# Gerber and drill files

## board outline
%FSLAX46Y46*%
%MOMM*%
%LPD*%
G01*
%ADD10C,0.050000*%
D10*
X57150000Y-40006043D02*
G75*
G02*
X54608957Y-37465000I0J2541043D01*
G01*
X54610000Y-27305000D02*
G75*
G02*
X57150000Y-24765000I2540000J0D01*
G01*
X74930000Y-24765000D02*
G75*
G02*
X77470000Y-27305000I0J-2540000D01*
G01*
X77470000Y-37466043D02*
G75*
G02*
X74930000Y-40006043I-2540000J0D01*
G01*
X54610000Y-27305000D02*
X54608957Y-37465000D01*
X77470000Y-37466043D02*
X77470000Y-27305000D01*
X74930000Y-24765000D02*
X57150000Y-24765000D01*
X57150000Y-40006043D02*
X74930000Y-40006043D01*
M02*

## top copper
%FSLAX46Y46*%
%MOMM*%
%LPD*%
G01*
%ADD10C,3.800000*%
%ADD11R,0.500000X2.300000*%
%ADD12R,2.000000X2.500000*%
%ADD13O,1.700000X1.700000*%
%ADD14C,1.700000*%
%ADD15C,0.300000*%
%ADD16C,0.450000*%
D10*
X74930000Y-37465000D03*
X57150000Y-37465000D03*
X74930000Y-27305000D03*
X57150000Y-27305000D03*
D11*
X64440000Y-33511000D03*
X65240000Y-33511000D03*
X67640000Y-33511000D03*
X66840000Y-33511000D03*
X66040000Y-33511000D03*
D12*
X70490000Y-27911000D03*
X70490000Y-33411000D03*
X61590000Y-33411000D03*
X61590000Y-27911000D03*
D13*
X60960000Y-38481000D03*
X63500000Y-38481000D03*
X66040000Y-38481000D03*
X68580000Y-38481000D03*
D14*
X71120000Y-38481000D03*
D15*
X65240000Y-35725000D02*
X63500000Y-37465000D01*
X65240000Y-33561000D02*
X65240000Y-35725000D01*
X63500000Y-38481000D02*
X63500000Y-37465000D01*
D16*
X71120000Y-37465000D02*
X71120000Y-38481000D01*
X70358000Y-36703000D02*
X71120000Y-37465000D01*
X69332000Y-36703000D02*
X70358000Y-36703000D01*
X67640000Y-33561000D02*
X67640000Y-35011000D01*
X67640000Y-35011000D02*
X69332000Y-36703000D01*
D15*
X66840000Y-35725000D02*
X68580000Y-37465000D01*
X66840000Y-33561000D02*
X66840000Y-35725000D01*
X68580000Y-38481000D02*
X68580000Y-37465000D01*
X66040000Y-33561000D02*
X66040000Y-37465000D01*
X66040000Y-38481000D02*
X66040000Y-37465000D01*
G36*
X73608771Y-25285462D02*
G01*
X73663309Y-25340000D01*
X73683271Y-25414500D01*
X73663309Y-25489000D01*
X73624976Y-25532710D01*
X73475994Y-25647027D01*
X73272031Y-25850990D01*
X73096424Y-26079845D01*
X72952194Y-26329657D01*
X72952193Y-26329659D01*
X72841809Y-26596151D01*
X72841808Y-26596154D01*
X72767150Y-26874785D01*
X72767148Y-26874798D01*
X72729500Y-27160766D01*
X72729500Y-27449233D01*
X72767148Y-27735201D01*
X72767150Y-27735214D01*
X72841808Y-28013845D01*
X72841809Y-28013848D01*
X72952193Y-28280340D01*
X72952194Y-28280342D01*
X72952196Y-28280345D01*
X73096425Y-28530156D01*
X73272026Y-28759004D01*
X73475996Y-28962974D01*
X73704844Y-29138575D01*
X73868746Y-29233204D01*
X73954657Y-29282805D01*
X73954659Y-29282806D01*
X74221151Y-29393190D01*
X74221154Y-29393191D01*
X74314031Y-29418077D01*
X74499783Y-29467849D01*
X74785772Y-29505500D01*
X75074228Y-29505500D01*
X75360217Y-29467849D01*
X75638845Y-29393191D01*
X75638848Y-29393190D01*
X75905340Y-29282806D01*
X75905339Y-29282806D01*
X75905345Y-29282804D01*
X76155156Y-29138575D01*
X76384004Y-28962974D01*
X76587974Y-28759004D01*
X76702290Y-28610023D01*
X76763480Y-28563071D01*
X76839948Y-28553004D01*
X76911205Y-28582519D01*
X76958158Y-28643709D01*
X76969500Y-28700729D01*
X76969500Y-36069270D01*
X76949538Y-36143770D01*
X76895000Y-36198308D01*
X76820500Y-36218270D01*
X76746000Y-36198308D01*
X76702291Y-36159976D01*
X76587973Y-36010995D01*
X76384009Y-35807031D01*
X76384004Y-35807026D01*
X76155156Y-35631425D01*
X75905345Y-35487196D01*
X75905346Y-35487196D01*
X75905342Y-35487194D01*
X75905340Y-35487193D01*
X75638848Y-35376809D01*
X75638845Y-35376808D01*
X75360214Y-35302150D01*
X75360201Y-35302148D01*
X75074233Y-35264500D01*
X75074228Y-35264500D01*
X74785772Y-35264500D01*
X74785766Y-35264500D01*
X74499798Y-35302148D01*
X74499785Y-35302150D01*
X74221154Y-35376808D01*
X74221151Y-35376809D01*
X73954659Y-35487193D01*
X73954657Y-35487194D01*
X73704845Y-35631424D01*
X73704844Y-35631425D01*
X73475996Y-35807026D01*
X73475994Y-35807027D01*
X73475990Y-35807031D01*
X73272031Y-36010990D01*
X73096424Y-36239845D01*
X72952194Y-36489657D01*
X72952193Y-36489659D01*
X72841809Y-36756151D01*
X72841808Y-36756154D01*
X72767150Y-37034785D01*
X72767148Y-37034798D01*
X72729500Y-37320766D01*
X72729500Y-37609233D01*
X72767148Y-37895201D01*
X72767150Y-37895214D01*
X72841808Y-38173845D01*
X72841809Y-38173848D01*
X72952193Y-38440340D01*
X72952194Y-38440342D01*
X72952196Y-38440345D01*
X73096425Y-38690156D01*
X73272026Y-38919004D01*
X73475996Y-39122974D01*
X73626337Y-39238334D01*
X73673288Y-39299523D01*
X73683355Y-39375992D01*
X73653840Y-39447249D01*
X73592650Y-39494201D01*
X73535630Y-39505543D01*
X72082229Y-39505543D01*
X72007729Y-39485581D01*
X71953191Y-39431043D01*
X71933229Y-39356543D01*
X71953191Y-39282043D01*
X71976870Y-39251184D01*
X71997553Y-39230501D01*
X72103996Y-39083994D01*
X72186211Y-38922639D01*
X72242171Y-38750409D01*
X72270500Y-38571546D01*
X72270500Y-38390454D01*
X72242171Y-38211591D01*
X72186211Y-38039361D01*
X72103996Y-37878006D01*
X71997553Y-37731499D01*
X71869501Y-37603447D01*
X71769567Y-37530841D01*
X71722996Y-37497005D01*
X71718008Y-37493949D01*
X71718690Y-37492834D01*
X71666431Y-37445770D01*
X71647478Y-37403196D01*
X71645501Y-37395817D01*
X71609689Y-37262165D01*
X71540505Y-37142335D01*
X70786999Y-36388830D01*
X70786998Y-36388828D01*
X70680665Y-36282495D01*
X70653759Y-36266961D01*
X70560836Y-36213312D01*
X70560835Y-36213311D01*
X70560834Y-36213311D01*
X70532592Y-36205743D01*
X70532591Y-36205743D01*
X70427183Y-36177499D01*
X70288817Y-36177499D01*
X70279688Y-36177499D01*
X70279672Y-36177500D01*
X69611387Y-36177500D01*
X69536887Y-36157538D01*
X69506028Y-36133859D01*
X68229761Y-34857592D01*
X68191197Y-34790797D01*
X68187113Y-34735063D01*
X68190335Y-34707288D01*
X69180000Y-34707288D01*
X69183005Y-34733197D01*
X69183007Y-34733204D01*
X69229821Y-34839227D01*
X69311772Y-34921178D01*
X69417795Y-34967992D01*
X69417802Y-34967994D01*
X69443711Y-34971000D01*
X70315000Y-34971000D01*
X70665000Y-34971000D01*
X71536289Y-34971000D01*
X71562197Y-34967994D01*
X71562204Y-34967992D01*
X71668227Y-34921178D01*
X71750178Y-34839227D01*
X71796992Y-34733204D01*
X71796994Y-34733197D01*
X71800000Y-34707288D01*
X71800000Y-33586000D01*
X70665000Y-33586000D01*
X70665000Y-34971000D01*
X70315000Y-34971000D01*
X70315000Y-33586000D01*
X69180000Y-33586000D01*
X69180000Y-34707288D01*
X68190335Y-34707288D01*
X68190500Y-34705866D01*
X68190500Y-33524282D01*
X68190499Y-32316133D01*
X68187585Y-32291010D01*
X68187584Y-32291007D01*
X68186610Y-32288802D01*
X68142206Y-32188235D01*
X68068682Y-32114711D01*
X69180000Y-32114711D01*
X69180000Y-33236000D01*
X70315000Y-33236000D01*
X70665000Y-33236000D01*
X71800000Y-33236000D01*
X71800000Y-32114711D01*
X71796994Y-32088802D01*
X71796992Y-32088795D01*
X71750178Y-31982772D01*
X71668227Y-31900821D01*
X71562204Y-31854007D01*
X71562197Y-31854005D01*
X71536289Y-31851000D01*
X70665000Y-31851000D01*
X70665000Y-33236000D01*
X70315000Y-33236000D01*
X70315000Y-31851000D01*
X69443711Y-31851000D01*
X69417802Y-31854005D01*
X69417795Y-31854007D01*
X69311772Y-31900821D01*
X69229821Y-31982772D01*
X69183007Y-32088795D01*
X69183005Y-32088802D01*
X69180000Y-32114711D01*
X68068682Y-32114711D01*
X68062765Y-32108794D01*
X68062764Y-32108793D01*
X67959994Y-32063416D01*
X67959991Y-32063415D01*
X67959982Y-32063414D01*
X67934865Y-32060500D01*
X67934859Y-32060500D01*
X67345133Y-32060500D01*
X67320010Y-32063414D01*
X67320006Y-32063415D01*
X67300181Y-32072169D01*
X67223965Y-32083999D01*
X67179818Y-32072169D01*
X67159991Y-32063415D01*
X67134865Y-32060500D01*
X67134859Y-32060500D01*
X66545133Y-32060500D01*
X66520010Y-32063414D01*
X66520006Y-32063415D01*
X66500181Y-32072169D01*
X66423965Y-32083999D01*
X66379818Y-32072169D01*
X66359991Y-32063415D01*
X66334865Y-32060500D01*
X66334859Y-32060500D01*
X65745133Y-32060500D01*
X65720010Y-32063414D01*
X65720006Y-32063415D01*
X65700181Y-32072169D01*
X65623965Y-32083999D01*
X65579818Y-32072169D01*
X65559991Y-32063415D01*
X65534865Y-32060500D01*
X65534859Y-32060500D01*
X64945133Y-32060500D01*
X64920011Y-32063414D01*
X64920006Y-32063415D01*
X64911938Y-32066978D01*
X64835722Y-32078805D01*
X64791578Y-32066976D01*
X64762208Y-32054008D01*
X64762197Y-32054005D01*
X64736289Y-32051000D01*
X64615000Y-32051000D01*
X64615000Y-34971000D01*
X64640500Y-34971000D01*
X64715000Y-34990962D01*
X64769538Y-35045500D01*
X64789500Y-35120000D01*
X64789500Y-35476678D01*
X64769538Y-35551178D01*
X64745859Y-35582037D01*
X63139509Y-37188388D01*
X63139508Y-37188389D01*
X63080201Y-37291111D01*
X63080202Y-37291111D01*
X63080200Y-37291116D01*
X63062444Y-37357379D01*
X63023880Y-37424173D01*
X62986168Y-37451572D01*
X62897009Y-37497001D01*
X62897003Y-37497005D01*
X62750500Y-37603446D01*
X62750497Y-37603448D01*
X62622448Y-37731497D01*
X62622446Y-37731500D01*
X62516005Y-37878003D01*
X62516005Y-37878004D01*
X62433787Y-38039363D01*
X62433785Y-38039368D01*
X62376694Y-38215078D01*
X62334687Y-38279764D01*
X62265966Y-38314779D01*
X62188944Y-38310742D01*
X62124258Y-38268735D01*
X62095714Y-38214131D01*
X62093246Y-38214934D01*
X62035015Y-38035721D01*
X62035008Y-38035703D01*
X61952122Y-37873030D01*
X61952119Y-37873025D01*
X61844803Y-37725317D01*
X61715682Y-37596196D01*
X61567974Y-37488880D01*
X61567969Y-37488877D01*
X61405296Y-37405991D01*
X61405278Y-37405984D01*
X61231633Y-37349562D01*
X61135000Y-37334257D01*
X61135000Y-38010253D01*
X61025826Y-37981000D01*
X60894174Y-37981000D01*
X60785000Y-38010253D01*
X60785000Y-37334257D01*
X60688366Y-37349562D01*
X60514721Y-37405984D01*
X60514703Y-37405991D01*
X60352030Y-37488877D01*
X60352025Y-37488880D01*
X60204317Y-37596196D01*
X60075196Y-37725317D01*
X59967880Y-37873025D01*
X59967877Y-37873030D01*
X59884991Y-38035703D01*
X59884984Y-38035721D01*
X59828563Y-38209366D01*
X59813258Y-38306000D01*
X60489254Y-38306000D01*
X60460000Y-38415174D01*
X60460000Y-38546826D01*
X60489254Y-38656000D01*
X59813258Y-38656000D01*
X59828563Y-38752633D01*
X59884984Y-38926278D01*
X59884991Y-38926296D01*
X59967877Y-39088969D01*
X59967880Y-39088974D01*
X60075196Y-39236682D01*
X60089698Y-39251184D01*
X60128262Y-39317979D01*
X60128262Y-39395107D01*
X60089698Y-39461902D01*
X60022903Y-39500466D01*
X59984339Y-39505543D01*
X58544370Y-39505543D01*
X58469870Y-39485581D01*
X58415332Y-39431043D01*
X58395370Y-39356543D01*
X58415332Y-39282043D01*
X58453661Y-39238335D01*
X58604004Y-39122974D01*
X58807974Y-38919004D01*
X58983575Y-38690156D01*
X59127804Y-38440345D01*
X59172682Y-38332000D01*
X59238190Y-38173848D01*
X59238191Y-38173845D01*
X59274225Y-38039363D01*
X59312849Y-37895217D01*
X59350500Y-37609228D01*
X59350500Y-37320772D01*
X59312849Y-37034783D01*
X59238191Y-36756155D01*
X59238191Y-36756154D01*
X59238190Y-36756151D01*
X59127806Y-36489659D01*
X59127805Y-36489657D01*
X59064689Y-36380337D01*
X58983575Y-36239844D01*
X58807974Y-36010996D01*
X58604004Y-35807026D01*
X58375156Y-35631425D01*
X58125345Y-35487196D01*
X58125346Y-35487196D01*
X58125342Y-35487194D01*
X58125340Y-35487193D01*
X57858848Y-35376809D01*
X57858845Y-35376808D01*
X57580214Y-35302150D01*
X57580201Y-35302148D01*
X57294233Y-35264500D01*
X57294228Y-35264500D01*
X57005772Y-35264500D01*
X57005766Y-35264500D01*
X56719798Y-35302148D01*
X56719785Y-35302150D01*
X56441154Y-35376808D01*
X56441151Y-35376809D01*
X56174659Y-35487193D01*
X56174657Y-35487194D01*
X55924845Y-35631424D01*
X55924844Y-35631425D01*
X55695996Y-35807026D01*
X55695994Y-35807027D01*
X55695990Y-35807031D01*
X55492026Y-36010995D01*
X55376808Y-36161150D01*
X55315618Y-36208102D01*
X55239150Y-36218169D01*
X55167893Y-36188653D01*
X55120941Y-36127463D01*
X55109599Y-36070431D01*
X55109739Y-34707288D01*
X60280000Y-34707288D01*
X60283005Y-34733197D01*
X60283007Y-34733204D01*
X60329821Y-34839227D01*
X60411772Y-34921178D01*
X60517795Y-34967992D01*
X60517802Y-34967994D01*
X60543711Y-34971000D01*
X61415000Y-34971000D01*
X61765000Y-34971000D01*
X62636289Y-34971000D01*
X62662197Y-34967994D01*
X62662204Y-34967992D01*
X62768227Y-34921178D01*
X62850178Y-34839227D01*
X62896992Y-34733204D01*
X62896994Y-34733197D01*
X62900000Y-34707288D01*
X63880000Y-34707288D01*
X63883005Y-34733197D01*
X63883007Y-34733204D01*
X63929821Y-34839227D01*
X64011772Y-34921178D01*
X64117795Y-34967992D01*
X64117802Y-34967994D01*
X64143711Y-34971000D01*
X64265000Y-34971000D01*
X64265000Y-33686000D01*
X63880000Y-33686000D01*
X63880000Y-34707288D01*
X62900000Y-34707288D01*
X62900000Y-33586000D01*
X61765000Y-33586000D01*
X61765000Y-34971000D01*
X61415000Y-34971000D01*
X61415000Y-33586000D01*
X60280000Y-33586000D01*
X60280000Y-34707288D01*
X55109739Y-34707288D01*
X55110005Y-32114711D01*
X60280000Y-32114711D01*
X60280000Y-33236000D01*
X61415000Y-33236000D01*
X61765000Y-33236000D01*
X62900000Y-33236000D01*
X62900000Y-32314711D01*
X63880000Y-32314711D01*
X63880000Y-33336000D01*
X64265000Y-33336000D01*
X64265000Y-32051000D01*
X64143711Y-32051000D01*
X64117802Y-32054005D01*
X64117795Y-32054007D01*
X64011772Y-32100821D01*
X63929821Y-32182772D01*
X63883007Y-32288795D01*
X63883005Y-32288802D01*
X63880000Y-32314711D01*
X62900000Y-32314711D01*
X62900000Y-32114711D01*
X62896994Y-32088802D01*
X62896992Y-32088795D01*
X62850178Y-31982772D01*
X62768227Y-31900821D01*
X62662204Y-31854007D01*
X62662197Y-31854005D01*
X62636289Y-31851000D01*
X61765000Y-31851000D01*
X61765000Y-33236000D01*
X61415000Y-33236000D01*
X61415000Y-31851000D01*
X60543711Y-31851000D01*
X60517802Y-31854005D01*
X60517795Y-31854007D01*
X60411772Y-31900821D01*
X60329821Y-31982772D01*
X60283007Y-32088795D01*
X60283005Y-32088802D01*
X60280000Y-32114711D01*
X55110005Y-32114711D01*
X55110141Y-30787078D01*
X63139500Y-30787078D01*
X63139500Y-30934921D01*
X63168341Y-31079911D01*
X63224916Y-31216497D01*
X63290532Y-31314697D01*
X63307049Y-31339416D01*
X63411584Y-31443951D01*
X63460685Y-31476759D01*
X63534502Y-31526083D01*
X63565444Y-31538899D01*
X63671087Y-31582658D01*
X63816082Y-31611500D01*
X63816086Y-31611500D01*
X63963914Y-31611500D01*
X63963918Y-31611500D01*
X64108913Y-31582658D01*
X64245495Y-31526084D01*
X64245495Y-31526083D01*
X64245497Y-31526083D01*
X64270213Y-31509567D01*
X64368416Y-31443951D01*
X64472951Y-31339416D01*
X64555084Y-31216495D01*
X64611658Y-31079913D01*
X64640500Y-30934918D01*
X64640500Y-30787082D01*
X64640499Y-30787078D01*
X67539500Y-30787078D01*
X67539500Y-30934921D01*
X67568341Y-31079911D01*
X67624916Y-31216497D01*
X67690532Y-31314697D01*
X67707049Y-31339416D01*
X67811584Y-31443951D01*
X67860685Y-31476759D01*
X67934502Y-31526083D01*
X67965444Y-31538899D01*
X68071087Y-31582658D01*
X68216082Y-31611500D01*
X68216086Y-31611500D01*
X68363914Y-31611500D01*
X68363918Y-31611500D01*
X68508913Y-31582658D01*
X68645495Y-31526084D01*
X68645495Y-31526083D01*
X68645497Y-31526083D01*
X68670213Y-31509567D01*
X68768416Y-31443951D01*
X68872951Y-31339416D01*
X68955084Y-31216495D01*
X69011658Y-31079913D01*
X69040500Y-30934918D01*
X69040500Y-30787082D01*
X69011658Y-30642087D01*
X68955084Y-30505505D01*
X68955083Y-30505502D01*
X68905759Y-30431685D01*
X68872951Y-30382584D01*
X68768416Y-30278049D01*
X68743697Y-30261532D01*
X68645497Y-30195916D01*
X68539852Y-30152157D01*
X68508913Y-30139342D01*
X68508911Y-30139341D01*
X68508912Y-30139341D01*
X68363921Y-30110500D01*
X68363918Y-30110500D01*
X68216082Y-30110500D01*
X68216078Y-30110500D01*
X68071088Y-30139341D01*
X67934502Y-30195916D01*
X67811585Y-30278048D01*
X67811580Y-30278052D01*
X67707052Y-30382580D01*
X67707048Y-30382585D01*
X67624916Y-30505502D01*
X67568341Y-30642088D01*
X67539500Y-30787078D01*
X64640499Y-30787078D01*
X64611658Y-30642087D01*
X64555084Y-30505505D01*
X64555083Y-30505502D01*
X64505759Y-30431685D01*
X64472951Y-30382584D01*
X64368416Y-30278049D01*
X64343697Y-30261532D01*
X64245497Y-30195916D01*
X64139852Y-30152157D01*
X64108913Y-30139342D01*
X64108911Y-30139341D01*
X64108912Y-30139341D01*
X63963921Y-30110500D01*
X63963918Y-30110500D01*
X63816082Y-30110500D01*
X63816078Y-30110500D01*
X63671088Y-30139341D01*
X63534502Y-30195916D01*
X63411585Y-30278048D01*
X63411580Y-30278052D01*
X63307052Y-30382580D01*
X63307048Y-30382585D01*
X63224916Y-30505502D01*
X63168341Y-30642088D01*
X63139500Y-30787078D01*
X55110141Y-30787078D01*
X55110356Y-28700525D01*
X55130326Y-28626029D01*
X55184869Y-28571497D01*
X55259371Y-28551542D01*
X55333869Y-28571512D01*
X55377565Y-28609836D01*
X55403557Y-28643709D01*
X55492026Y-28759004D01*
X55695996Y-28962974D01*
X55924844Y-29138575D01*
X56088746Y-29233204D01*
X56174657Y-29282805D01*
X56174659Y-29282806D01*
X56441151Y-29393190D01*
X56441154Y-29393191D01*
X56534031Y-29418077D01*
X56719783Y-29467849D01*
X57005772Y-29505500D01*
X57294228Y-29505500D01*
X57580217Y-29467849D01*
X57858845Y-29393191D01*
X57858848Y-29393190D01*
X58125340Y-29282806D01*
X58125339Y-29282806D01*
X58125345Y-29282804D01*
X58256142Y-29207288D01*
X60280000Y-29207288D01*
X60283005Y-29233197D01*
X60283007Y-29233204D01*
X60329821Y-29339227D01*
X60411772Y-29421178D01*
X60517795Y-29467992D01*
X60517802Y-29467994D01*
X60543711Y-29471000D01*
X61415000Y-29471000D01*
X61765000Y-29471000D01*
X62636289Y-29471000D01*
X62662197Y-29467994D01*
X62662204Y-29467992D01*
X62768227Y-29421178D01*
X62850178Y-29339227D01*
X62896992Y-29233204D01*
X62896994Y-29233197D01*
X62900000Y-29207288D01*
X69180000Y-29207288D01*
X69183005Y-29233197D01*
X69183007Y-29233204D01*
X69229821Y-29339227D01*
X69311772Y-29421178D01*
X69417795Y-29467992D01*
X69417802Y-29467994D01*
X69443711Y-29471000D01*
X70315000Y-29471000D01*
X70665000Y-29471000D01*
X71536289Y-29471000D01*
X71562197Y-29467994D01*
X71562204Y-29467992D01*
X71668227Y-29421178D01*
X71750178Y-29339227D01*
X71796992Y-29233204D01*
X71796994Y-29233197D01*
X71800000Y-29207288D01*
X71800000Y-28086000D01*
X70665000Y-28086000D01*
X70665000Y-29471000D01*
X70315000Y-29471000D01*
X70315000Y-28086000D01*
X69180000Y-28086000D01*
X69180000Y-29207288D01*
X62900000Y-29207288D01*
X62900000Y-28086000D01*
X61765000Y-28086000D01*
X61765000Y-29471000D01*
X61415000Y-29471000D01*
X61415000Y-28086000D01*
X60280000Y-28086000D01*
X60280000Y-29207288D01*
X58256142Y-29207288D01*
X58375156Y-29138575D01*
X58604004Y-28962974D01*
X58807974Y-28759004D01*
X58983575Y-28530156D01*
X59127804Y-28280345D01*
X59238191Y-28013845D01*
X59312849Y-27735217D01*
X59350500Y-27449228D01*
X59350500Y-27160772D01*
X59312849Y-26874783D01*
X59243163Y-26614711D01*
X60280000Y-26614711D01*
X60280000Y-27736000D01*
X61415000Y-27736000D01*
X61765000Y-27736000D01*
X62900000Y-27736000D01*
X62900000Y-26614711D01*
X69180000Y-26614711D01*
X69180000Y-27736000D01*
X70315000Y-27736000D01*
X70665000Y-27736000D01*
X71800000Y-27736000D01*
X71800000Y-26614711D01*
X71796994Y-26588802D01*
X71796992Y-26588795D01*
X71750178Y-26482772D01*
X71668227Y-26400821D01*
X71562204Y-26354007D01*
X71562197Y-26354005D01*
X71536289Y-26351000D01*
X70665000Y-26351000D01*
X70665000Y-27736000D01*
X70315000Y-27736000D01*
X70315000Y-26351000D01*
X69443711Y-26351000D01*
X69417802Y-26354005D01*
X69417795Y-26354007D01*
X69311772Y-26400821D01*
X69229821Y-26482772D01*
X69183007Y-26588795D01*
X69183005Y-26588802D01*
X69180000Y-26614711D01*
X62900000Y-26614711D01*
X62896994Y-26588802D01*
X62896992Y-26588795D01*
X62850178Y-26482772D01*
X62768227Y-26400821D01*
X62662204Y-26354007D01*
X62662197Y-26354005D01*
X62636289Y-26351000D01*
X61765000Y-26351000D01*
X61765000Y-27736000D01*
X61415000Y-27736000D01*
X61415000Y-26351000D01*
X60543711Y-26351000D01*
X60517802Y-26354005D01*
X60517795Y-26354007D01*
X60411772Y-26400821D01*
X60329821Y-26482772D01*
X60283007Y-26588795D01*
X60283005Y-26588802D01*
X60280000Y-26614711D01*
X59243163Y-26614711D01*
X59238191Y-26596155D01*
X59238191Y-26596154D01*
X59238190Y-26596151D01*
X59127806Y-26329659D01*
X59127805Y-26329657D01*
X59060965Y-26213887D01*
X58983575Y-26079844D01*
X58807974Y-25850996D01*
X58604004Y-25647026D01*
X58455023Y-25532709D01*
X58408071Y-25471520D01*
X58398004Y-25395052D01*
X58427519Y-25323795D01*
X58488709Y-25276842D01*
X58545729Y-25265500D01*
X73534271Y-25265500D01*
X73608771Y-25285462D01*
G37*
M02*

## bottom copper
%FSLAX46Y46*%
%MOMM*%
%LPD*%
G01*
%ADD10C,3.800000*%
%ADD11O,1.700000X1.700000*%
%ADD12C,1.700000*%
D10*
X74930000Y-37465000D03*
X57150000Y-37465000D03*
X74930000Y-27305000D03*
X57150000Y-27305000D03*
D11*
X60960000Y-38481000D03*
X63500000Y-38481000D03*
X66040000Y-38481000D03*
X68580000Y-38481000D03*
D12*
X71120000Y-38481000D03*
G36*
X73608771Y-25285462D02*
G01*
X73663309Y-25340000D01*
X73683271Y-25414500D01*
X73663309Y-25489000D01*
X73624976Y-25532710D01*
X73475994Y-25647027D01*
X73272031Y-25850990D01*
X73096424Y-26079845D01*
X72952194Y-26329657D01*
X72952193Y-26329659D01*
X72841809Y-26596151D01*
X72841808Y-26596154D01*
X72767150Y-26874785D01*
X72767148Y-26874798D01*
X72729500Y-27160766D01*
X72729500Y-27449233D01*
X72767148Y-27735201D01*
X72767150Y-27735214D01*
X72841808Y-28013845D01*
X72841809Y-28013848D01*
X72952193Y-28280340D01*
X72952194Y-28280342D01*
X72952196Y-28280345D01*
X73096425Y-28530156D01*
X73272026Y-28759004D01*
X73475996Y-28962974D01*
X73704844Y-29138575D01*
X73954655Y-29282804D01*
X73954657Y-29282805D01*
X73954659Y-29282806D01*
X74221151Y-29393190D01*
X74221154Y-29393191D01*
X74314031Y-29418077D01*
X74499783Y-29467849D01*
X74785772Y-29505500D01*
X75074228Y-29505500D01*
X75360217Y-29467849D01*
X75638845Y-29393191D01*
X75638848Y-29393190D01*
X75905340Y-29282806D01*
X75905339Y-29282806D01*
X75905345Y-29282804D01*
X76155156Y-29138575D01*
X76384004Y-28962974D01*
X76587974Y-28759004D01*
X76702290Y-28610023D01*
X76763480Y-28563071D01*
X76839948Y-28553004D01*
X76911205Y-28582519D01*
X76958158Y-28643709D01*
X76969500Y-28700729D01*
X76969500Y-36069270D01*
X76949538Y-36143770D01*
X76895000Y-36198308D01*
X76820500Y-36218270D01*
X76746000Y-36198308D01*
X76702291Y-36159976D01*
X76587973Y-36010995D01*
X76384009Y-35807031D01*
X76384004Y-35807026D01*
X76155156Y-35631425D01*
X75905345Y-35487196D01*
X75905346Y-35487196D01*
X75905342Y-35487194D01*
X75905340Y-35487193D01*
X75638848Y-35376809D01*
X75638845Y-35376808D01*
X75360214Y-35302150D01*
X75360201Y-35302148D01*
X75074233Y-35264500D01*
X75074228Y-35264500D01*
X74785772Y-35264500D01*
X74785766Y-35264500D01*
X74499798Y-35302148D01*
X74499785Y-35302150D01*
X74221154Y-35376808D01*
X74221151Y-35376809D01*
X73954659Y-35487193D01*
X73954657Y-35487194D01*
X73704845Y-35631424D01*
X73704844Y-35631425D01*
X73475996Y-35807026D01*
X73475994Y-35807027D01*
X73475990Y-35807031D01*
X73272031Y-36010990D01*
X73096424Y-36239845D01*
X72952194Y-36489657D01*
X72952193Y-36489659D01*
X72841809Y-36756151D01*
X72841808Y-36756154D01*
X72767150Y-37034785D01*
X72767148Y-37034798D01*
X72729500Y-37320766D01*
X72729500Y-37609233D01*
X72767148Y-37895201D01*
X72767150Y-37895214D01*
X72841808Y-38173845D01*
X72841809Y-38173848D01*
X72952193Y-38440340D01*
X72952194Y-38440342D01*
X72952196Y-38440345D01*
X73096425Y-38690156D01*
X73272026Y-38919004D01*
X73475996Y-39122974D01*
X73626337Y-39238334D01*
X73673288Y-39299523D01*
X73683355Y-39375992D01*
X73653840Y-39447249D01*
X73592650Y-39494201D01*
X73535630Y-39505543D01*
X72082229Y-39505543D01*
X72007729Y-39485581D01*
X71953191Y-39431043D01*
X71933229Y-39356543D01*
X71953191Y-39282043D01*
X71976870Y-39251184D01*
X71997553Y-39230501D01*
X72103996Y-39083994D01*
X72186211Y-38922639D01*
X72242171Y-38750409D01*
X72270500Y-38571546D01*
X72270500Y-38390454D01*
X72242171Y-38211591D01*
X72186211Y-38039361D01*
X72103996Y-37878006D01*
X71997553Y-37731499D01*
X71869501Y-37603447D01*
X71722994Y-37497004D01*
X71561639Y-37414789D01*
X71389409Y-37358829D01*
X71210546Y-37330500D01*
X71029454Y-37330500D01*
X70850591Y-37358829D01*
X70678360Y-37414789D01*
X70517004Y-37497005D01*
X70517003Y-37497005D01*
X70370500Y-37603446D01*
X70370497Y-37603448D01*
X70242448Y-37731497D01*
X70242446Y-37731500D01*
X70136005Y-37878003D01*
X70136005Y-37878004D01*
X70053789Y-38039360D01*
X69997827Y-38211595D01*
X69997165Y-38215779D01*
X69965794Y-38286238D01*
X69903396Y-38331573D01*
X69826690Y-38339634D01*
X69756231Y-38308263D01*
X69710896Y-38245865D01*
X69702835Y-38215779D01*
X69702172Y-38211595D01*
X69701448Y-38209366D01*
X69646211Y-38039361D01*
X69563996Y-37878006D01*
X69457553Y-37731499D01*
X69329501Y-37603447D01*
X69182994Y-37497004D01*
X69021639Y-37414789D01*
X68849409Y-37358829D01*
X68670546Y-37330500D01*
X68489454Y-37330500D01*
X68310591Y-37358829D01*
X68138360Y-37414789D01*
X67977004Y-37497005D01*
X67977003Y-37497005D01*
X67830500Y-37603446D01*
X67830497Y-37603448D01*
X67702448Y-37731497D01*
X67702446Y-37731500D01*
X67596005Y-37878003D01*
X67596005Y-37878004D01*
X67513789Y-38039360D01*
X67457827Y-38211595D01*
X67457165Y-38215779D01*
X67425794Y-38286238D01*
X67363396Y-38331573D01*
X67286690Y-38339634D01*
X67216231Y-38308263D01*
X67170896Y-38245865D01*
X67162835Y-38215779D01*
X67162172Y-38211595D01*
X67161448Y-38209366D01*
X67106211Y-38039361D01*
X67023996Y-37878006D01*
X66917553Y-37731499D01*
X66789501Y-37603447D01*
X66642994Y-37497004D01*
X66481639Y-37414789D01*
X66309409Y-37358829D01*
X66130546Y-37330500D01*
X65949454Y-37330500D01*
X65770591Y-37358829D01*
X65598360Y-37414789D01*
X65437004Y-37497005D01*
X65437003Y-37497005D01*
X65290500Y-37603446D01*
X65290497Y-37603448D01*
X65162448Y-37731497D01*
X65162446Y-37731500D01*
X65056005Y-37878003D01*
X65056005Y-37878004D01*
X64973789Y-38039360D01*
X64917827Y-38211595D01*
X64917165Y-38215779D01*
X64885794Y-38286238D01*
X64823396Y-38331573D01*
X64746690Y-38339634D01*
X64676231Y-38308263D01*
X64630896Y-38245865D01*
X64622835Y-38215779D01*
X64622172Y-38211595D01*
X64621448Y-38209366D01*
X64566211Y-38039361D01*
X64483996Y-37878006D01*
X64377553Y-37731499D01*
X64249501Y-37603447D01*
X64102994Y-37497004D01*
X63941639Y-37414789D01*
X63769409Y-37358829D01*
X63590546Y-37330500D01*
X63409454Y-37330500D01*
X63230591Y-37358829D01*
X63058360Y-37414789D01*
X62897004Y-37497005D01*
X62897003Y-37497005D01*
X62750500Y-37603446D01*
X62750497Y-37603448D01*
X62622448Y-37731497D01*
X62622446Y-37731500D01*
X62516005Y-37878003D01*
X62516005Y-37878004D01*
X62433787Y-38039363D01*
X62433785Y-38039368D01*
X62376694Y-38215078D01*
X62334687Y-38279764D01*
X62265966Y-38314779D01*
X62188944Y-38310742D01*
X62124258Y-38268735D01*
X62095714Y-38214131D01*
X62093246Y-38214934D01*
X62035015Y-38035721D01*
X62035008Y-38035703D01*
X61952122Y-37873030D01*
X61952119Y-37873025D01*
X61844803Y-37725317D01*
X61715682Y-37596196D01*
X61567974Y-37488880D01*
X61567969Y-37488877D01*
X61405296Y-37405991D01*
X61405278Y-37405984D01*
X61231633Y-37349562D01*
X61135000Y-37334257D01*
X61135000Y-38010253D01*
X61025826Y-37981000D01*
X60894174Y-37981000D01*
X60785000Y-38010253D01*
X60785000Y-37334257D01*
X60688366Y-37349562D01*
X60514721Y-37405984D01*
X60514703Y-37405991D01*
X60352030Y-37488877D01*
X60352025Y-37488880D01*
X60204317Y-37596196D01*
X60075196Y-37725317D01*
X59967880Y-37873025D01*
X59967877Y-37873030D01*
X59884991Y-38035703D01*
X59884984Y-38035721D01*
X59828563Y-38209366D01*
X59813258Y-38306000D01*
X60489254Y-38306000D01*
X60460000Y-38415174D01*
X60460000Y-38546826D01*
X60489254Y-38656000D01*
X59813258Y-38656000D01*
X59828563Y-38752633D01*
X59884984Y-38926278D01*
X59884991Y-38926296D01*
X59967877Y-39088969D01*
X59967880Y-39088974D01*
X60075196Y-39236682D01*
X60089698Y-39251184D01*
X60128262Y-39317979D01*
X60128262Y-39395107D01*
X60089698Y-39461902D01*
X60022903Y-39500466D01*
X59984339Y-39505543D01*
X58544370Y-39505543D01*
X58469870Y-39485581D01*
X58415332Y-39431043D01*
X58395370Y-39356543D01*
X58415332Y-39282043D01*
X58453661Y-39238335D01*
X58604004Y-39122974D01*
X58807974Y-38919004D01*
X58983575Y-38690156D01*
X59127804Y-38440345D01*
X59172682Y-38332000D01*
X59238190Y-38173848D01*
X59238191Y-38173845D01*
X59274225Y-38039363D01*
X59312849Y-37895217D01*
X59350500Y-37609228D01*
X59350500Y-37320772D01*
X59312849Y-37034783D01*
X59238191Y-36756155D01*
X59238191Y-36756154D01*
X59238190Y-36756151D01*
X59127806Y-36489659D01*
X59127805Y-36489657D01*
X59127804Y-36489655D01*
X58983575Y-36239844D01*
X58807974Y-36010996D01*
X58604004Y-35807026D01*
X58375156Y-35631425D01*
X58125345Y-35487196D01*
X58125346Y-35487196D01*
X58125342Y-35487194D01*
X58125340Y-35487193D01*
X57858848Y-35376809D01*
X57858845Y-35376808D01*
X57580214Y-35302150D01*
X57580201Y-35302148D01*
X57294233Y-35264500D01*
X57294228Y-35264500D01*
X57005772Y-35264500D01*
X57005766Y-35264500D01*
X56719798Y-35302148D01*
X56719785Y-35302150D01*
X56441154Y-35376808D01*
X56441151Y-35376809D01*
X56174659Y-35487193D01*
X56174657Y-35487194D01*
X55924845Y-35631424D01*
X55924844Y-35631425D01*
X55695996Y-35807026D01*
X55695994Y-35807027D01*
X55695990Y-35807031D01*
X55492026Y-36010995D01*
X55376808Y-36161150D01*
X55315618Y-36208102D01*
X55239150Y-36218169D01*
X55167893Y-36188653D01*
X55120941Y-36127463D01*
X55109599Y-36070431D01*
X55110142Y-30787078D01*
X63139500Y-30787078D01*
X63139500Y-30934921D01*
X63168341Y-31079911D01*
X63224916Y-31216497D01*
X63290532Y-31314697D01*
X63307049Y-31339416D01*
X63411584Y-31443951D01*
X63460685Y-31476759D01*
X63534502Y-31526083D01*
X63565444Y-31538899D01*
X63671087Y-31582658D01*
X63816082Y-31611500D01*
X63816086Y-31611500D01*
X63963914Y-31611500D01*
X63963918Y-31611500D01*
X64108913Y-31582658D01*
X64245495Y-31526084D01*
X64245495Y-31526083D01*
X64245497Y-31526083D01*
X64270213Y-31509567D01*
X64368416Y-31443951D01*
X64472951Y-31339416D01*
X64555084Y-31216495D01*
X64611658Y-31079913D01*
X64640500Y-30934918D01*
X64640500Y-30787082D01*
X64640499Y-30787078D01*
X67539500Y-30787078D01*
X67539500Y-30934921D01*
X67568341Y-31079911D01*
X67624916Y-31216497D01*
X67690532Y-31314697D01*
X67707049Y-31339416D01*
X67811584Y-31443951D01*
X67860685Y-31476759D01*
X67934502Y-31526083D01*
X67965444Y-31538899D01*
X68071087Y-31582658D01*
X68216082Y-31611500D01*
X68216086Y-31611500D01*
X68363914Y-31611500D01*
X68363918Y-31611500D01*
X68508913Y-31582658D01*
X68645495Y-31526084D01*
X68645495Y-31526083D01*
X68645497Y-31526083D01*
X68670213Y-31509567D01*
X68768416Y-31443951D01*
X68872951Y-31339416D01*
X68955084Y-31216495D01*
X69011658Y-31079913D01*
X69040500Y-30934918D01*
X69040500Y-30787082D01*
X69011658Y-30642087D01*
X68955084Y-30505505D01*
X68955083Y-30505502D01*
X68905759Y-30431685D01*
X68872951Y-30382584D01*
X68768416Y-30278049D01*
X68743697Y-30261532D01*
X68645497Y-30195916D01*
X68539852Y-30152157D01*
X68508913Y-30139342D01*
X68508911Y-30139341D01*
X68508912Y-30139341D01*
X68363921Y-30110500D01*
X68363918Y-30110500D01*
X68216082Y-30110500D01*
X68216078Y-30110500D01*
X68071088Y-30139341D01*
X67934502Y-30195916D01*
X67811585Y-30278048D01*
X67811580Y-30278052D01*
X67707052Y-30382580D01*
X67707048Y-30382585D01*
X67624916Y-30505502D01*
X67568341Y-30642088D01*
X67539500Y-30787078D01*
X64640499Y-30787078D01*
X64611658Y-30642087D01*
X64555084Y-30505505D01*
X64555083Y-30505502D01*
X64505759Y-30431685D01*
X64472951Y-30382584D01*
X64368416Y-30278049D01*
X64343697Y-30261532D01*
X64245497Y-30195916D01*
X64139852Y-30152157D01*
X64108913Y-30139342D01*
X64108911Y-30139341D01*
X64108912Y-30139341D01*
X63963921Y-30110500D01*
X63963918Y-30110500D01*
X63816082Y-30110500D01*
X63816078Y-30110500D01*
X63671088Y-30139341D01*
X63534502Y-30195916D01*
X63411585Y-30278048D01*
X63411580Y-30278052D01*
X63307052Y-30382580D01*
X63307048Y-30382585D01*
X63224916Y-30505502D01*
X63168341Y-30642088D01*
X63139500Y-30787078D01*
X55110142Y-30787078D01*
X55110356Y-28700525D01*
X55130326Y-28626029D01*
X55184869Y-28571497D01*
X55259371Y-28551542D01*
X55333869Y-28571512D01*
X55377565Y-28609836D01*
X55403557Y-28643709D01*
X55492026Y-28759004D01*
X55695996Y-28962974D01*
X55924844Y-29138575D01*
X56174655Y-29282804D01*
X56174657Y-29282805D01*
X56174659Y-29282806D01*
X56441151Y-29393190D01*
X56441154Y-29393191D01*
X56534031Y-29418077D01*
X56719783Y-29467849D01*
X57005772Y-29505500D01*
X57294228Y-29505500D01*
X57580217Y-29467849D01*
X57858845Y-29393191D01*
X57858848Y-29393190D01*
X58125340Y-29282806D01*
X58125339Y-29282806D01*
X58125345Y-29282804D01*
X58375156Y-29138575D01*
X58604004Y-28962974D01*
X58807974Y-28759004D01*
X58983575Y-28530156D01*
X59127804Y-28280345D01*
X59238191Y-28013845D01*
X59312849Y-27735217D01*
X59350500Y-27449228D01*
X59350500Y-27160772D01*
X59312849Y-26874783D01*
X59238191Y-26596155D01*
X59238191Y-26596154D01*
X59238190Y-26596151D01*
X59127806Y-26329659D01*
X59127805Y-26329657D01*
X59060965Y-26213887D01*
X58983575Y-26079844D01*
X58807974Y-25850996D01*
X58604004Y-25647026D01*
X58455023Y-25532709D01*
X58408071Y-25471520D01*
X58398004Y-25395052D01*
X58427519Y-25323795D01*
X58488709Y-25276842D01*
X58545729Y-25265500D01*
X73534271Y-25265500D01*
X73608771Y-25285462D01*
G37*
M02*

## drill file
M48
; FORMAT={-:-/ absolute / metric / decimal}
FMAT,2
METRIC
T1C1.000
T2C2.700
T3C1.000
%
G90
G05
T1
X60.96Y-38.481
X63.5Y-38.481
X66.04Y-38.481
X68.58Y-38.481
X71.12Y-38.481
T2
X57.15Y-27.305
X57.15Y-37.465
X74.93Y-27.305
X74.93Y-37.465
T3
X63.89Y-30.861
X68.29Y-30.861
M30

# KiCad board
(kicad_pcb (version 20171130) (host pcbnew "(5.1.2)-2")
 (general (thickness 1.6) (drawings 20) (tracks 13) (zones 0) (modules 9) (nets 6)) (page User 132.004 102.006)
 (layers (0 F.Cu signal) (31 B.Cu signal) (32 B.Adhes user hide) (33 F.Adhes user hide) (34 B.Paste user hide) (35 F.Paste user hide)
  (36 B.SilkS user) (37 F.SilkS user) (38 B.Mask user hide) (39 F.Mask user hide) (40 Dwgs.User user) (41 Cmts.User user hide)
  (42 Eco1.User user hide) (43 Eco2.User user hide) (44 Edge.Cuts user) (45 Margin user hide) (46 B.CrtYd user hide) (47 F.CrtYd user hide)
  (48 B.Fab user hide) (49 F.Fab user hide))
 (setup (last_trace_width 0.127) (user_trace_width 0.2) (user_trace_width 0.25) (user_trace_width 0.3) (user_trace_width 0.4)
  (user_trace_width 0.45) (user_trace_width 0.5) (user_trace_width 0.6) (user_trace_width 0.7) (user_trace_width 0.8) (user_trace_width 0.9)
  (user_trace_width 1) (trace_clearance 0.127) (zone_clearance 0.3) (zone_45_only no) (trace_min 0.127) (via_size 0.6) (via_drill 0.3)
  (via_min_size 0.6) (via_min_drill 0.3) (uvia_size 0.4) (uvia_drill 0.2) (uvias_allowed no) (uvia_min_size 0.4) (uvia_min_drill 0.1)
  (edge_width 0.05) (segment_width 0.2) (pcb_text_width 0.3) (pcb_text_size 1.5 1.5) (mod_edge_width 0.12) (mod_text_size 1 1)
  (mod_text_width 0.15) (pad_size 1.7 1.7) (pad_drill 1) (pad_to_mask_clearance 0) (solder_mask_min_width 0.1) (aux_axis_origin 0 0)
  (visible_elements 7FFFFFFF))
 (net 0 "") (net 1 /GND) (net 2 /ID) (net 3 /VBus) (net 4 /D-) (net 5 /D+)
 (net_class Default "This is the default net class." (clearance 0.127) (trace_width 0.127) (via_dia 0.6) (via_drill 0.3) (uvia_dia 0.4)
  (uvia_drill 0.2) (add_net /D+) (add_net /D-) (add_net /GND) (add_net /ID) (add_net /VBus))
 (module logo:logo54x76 (layer F.Cu) (at 57.0865 32.385)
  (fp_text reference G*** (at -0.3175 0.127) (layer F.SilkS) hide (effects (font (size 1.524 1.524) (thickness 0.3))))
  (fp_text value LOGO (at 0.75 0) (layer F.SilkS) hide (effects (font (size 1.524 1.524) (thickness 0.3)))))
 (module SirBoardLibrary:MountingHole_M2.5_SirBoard (layer F.Cu) (at 74.93 37.465)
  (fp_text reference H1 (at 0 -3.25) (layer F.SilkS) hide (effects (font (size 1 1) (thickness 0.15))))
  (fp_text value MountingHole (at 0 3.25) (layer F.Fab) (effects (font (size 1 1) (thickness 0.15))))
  (pad 1 thru_hole circle (at 0 0) (size 3.8 3.8) (drill 2.7) (layers *.Cu *.Mask)))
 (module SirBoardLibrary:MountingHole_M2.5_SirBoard (layer F.Cu) (at 57.15 37.465)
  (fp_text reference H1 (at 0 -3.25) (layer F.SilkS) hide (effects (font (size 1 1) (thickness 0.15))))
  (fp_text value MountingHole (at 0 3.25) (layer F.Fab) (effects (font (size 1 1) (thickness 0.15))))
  (pad 1 thru_hole circle (at 0 0) (size 3.8 3.8) (drill 2.7) (layers *.Cu *.Mask)))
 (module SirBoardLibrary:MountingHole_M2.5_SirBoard (layer F.Cu) (at 74.93 27.305)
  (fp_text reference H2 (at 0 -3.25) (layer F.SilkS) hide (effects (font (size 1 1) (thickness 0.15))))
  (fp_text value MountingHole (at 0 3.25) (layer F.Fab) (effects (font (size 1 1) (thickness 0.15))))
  (pad 1 thru_hole circle (at 0 0) (size 3.8 3.8) (drill 2.7) (layers *.Cu *.Mask)))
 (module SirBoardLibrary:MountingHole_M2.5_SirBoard (layer F.Cu) (at 57.15 27.305)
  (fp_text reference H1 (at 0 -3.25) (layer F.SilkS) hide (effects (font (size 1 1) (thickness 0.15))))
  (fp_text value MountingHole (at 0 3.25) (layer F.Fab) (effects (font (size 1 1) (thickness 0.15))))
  (pad 1 thru_hole circle (at 0 0) (size 3.8 3.8) (drill 2.7) (layers *.Cu *.Mask)))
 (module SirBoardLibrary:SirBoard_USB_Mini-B (layer F.Cu) (at 66.04 30.861 180)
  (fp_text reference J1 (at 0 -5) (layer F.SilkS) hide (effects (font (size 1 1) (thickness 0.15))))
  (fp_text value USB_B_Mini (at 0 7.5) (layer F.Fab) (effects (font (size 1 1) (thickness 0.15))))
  (pad 5 smd rect (at 1.6 -2.65) (size 0.5 2.3) (layers F.Cu F.Paste F.Mask) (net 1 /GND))
  (pad 4 smd rect (at 0.8 -2.65) (size 0.5 2.3) (layers F.Cu F.Paste F.Mask) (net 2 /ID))
  (pad 1 smd rect (at -1.6 -2.65) (size 0.5 2.3) (layers F.Cu F.Paste F.Mask) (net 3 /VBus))
  (pad 2 smd rect (at -0.8 -2.65) (size 0.5 2.3) (layers F.Cu F.Paste F.Mask) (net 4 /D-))
  (pad 3 smd rect (at 0 -2.65) (size 0.5 2.3) (layers F.Cu F.Paste F.Mask) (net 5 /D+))
  (pad "" np_thru_hole circle (at -2.25 0) (size 1 1) (drill 1) (layers *.Cu *.Mask))
  (pad "" np_thru_hole circle (at 2.15 0) (size 1 1) (drill 1) (layers *.Cu *.Mask))
  (pad 6 smd rect (at -4.45 2.95) (size 2 2.5) (layers F.Cu F.Paste F.Mask) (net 1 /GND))
  (pad 6 smd rect (at -4.45 -2.55) (size 2 2.5) (layers F.Cu F.Paste F.Mask) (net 1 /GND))
  (pad 6 smd rect (at 4.45 -2.55) (size 2 2.5) (layers F.Cu F.Paste F.Mask) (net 1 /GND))
  (pad 6 smd rect (at 4.45 2.95) (size 2 2.5) (layers F.Cu F.Paste F.Mask) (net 1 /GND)))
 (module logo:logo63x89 (layer B.Cu) (at 66.04 28.448 180)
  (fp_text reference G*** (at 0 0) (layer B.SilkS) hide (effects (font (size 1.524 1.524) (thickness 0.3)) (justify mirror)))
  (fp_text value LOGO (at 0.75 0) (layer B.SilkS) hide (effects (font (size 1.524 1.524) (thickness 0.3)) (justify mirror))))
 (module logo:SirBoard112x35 (layer B.Cu) (at 66.04 33.655 180)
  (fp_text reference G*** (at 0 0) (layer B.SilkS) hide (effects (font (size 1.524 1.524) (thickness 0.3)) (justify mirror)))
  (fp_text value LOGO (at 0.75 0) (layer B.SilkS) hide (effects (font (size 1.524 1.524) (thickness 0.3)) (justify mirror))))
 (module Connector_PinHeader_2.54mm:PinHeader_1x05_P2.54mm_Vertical (layer B.Cu) (at 71.12 38.481 90)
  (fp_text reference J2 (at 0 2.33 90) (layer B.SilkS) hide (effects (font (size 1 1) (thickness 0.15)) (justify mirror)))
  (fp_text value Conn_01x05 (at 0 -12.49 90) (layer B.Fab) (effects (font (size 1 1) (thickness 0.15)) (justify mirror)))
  (pad 5 thru_hole oval (at 0 -10.16 90) (size 1.7 1.7) (drill 1) (layers *.Cu *.Mask) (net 1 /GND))
  (pad 4 thru_hole oval (at 0 -7.62 90) (size 1.7 1.7) (drill 1) (layers *.Cu *.Mask) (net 2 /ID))
  (pad 3 thru_hole oval (at 0 -5.08 90) (size 1.7 1.7) (drill 1) (layers *.Cu *.Mask) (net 5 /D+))
  (pad 2 thru_hole oval (at 0 -2.54 90) (size 1.7 1.7) (drill 1) (layers *.Cu *.Mask) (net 4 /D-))
  (pad 1 thru_hole circle (at 0 0 90) (size 1.7 1.7) (drill 1) (layers *.Cu *.Mask) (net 3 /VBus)))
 (gr_arc (start 57.15 37.465) (end 54.608957 37.465) (angle -90) (layer Edge.Cuts) (width 0.05))
 (gr_arc (start 57.15 27.305) (end 57.15 24.765) (angle -90) (layer Edge.Cuts) (width 0.05))
 (gr_arc (start 74.93 27.305) (end 77.47 27.305) (angle -90) (layer Edge.Cuts) (width 0.05))
 (gr_arc (start 74.93 37.466043) (end 74.93 40.006043) (angle -90) (layer Edge.Cuts) (width 0.05))
 (gr_line (start 54.61 27.305) (end 54.608957 37.465) (layer Edge.Cuts) (width 0.05))
 (gr_line (start 77.47 37.466043) (end 77.47 27.305) (layer Edge.Cuts) (width 0.05))
 (gr_line (start 74.93 24.765) (end 57.15 24.765) (layer Edge.Cuts) (width 0.05))
 (gr_line (start 57.15 40.006043) (end 74.93 40.006043) (layer Edge.Cuts) (width 0.05))
 (segment (start 65.24 35.725) (end 63.5 37.465) (width 0.3) (layer F.Cu) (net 2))
 (segment (start 65.24 33.561) (end 65.24 35.725) (width 0.3) (layer F.Cu) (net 2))
 (segment (start 63.5 38.481) (end 63.5 37.465) (width 0.3) (layer F.Cu) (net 2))
 (segment (start 71.12 37.465) (end 71.12 38.481) (width 0.45) (layer F.Cu) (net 3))
 (segment (start 70.358 36.703) (end 71.12 37.465) (width 0.45) (layer F.Cu) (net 3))
 (segment (start 69.332 36.703) (end 70.358 36.703) (width 0.45) (layer F.Cu) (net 3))
 (segment (start 67.64 33.561) (end 67.64 35.011) (width 0.45) (layer F.Cu) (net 3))
 (segment (start 67.64 35.011) (end 69.332 36.703) (width 0.45) (layer F.Cu) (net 3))
 (segment (start 66.84 35.725) (end 68.58 37.465) (width 0.3) (layer F.Cu) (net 4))
 (segment (start 66.84 33.561) (end 66.84 35.725) (width 0.3) (layer F.Cu) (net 4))
 (segment (start 68.58 38.481) (end 68.58 37.465) (width 0.3) (layer F.Cu) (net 4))
 (segment (start 66.04 33.561) (end 66.04 37.465) (width 0.3) (layer F.Cu) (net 5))
 (segment (start 66.04 38.481) (end 66.04 37.465) (width 0.3) (layer F.Cu) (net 5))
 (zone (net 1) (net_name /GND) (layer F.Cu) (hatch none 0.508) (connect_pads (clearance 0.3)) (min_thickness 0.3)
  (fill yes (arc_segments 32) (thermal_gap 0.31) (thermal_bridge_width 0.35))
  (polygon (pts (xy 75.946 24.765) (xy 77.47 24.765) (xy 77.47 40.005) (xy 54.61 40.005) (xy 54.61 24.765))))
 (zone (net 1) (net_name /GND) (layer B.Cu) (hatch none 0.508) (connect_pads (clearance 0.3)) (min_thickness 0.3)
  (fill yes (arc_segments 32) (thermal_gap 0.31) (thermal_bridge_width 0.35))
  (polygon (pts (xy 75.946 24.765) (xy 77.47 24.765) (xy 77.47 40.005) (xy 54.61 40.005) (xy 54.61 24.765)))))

